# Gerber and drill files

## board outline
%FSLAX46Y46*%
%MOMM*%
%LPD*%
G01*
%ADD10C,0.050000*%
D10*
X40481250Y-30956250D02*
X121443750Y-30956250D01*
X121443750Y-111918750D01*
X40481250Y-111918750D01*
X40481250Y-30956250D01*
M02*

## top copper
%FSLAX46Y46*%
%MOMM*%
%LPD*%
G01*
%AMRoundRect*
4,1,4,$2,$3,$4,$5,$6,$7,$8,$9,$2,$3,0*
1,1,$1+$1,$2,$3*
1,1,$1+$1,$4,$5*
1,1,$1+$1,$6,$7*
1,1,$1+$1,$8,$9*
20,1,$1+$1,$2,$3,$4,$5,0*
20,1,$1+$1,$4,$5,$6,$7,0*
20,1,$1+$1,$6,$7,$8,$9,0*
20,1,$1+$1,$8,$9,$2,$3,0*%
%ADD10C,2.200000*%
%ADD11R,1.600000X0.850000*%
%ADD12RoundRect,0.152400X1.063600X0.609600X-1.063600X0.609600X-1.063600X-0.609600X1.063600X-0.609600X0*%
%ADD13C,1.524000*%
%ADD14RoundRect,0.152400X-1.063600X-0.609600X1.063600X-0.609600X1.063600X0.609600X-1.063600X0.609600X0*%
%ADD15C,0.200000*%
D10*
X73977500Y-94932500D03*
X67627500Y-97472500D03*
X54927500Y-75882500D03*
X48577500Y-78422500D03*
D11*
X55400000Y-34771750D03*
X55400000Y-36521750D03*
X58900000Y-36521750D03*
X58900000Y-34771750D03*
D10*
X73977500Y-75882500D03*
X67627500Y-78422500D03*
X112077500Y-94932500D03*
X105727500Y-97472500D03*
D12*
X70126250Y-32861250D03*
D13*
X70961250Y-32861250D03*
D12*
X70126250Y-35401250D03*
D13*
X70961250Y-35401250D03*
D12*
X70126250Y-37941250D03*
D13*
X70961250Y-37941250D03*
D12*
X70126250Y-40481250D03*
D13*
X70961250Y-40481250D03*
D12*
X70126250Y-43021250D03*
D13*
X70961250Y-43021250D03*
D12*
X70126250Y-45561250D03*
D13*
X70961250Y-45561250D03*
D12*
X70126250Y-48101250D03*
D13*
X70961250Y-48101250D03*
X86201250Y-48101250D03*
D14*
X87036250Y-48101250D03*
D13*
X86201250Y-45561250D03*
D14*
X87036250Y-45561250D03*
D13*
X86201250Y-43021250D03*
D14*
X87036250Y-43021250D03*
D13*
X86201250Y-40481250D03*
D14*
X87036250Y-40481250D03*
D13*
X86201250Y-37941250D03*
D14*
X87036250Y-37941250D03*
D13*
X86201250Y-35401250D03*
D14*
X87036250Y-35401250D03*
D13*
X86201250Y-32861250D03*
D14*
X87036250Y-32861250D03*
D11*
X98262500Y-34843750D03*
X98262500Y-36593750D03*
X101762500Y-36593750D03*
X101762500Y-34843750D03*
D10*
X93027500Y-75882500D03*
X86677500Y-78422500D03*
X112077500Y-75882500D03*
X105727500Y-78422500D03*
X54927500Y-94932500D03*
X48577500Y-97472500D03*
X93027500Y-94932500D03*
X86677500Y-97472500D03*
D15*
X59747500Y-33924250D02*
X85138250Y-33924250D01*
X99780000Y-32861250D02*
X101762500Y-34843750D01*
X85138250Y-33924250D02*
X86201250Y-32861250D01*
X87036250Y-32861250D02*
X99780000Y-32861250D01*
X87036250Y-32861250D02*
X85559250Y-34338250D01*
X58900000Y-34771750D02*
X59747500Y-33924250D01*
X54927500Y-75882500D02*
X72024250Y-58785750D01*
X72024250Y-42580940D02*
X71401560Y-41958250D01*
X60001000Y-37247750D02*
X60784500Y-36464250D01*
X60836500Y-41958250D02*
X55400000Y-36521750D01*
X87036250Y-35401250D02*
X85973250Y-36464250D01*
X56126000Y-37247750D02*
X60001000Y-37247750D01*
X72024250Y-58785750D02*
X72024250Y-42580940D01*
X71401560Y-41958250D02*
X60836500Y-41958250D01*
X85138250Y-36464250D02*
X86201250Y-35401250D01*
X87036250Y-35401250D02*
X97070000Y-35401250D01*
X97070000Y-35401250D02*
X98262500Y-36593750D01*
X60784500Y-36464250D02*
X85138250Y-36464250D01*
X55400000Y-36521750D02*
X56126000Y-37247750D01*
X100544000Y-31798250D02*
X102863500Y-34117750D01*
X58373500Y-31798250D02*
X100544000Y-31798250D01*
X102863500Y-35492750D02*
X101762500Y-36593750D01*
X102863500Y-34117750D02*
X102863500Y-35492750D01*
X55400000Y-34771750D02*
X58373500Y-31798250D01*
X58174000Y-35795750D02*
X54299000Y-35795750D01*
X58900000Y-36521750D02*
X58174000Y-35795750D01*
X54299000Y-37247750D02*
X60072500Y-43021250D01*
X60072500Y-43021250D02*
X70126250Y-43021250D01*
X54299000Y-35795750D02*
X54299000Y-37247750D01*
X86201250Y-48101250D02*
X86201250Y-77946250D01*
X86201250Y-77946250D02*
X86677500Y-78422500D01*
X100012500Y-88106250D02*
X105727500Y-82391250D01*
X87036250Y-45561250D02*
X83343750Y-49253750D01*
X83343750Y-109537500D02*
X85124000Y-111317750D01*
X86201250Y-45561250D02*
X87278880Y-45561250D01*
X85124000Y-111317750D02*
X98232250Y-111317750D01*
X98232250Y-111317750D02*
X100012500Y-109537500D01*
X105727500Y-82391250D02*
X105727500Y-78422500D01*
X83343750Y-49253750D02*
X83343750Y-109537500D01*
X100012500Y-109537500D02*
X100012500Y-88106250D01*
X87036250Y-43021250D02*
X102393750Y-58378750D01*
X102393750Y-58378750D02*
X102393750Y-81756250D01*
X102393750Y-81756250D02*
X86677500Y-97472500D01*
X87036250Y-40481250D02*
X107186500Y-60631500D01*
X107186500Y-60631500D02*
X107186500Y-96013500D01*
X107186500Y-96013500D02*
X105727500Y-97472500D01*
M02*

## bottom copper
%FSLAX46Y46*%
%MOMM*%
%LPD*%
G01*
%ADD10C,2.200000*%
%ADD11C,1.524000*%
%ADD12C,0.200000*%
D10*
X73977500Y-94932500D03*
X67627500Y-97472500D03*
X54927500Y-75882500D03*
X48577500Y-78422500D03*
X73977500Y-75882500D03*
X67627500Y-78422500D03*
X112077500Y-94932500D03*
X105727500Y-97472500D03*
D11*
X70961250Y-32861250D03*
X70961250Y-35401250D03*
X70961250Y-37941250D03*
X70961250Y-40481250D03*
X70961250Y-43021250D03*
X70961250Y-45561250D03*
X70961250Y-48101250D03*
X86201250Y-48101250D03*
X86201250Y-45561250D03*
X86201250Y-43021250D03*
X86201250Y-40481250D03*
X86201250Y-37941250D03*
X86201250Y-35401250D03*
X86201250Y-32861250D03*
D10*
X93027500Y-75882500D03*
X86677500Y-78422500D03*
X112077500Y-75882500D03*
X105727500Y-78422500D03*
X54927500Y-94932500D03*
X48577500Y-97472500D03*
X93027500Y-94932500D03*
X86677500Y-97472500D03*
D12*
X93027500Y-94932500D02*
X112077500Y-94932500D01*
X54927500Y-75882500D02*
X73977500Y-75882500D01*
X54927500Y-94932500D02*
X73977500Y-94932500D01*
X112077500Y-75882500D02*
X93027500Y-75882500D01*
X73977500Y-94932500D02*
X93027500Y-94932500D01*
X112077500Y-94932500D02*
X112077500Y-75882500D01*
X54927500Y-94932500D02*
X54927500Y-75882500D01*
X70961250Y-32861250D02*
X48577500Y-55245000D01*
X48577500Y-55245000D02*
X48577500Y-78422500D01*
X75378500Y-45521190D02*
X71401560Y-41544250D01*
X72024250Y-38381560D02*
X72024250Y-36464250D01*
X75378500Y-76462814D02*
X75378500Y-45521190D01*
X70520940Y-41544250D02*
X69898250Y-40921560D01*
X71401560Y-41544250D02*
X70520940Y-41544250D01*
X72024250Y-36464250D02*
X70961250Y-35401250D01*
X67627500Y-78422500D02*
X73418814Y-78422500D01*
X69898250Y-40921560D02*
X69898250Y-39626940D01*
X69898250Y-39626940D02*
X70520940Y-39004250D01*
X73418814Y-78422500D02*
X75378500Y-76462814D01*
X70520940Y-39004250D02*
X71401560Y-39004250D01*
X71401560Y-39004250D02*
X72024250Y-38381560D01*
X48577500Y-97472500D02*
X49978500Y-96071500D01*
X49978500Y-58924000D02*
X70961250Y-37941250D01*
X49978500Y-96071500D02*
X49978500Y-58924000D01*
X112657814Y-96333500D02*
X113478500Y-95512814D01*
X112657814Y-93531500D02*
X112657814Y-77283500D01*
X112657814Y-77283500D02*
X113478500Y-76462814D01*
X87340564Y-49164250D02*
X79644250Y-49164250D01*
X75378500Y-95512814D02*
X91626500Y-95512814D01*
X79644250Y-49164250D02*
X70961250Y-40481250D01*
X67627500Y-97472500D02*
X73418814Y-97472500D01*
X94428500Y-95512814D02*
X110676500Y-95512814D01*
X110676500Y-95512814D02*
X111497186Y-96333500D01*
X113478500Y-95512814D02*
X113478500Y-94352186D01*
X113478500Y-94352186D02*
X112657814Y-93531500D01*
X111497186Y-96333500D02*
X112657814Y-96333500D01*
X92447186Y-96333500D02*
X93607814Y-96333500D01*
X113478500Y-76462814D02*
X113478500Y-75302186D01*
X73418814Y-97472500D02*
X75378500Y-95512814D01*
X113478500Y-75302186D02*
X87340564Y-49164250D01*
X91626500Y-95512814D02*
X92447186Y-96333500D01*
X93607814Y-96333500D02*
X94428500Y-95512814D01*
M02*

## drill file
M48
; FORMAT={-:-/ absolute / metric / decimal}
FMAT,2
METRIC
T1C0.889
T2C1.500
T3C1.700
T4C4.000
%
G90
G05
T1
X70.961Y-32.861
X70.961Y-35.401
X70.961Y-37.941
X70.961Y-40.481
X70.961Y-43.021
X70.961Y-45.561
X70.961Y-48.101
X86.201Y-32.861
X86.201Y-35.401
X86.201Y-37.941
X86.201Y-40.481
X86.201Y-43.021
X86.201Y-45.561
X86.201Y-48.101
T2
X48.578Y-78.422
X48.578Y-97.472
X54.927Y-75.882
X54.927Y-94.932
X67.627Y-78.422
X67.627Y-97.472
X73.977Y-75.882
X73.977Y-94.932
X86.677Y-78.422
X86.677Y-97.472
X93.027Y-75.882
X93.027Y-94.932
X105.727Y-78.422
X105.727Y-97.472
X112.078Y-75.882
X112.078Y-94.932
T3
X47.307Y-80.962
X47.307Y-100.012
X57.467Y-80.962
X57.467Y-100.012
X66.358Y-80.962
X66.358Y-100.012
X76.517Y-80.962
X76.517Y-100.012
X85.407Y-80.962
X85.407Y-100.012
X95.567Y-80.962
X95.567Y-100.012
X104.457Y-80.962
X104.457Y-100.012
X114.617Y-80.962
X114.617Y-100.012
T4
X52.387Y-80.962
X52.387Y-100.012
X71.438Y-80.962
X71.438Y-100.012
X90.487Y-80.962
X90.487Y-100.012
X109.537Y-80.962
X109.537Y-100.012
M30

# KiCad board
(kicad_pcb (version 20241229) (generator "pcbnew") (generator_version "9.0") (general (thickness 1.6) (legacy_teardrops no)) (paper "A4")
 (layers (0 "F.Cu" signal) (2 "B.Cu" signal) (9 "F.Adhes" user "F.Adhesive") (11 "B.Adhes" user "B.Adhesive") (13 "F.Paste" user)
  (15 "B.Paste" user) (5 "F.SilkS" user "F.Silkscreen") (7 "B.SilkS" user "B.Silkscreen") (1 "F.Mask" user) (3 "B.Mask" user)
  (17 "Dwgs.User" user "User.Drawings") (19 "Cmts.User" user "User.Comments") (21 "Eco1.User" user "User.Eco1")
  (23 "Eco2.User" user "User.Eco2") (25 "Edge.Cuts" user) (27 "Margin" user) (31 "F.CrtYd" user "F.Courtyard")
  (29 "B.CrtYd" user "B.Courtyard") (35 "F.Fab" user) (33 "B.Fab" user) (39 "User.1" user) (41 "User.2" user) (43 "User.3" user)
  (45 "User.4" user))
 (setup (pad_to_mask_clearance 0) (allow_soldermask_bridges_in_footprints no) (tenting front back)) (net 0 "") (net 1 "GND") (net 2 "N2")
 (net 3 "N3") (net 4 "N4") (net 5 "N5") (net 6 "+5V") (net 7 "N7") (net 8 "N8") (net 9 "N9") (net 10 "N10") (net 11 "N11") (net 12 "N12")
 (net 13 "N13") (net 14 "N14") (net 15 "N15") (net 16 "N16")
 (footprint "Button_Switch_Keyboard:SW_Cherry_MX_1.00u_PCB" (layer "F.Cu") (at 73.9775 94.9325)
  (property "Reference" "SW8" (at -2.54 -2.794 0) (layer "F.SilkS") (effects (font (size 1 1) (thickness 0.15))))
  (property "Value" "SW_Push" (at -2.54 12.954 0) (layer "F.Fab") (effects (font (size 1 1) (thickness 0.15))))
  (pad "" np_thru_hole circle (at -7.62 5.08) (size 1.7 1.7) (drill 1.7) (layers "*.Cu" "*.Mask"))
  (pad "" np_thru_hole circle (at -2.54 5.08) (size 4 4) (drill 4) (layers "*.Cu" "*.Mask"))
  (pad "" np_thru_hole circle (at 2.54 5.08) (size 1.7 1.7) (drill 1.7) (layers "*.Cu" "*.Mask"))
  (pad "1" thru_hole circle (at 0 0) (size 2.2 2.2) (drill 1.5) (layers "*.Cu" "*.Mask") (remove_unused_layers no) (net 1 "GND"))
  (pad "2" thru_hole circle (at -6.35 2.54) (size 2.2 2.2) (drill 1.5) (layers "*.Cu" "*.Mask") (remove_unused_layers no) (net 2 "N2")))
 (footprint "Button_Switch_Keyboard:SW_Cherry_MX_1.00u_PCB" (layer "F.Cu") (at 54.9275 75.8825)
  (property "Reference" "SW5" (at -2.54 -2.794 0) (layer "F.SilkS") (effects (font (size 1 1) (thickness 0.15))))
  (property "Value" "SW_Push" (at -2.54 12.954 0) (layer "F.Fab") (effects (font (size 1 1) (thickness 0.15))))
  (pad "" np_thru_hole circle (at -7.62 5.08) (size 1.7 1.7) (drill 1.7) (layers "*.Cu" "*.Mask"))
  (pad "" np_thru_hole circle (at -2.54 5.08) (size 4 4) (drill 4) (layers "*.Cu" "*.Mask"))
  (pad "" np_thru_hole circle (at 2.54 5.08) (size 1.7 1.7) (drill 1.7) (layers "*.Cu" "*.Mask"))
  (pad "1" thru_hole circle (at 0 0) (size 2.2 2.2) (drill 1.5) (layers "*.Cu" "*.Mask") (remove_unused_layers no) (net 1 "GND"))
  (pad "2" thru_hole circle (at -6.35 2.54) (size 2.2 2.2) (drill 1.5) (layers "*.Cu" "*.Mask") (remove_unused_layers no) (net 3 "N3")))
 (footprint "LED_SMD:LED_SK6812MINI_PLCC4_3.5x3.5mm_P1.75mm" (layer "F.Cu") (at 57.15 35.64675)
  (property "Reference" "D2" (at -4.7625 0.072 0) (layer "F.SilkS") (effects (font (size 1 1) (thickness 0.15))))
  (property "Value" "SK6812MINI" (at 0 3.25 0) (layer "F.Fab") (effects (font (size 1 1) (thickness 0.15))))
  (pad "1" smd rect (at -1.75 -0.875) (size 1.6 0.85) (layers "F.Cu" "F.Mask" "F.Paste") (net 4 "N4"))
  (pad "2" smd rect (at -1.75 0.875) (size 1.6 0.85) (layers "F.Cu" "F.Mask" "F.Paste") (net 1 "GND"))
  (pad "3" smd rect (at 1.75 0.875) (size 1.6 0.85) (layers "F.Cu" "F.Mask" "F.Paste") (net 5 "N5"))
  (pad "4" smd rect (at 1.75 -0.875) (size 1.6 0.85) (layers "F.Cu" "F.Mask" "F.Paste") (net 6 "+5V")))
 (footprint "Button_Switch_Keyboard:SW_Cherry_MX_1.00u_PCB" (layer "F.Cu") (at 73.9775 75.8825)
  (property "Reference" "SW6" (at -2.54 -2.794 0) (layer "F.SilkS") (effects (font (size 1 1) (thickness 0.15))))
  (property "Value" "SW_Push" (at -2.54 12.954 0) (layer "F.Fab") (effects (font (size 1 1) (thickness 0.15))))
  (pad "" np_thru_hole circle (at -7.62 5.08) (size 1.7 1.7) (drill 1.7) (layers "*.Cu" "*.Mask"))
  (pad "" np_thru_hole circle (at -2.54 5.08) (size 4 4) (drill 4) (layers "*.Cu" "*.Mask"))
  (pad "" np_thru_hole circle (at 2.54 5.08) (size 1.7 1.7) (drill 1.7) (layers "*.Cu" "*.Mask"))
  (pad "1" thru_hole circle (at 0 0) (size 2.2 2.2) (drill 1.5) (layers "*.Cu" "*.Mask") (remove_unused_layers no) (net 1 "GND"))
  (pad "2" thru_hole circle (at -6.35 2.54) (size 2.2 2.2) (drill 1.5) (layers "*.Cu" "*.Mask") (remove_unused_layers no) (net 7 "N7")))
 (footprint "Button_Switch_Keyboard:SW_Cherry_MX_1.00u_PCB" (layer "F.Cu") (at 112.0775 94.9325)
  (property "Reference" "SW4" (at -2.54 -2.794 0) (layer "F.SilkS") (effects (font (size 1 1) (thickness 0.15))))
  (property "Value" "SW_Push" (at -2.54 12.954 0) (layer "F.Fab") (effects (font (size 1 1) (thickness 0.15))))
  (pad "" np_thru_hole circle (at -7.62 5.08) (size 1.7 1.7) (drill 1.7) (layers "*.Cu" "*.Mask"))
  (pad "" np_thru_hole circle (at -2.54 5.08) (size 4 4) (drill 4) (layers "*.Cu" "*.Mask"))
  (pad "" np_thru_hole circle (at 2.54 5.08) (size 1.7 1.7) (drill 1.7) (layers "*.Cu" "*.Mask"))
  (pad "1" thru_hole circle (at 0 0) (size 2.2 2.2) (drill 1.5) (layers "*.Cu" "*.Mask") (remove_unused_layers no) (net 1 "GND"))
  (pad "2" thru_hole circle (at -6.35 2.54) (size 2.2 2.2) (drill 1.5) (layers "*.Cu" "*.Mask") (remove_unused_layers no) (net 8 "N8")))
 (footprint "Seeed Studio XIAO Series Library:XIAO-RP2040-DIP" (layer "F.Cu") (at 78.58125 40.48125)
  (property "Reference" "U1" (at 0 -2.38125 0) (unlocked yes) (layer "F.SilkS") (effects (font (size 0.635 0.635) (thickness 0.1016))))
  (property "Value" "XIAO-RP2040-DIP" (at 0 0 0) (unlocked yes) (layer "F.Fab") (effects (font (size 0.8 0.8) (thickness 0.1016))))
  (pad "1" smd roundrect (at -8.455 -7.62 180) (size 2.432 1.524) (layers "F.Cu" "F.Mask") (roundrect_rratio 0.1) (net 3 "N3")
   (thermal_bridge_angle 45))
  (pad "1" thru_hole circle (at -7.62 -7.62 180) (size 1.524 1.524) (drill 0.889) (layers "*.Cu" "*.Mask") (remove_unused_layers no)
   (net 3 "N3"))
  (pad "2" smd roundrect (at -8.455 -5.08 180) (size 2.432 1.524) (layers "F.Cu" "F.Mask") (roundrect_rratio 0.1) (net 7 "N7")
   (thermal_bridge_angle 45))
  (pad "2" thru_hole circle (at -7.62 -5.08 180) (size 1.524 1.524) (drill 0.889) (layers "*.Cu" "*.Mask") (remove_unused_layers no)
   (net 7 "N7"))
  (pad "3" smd roundrect (at -8.455 -2.54 180) (size 2.432 1.524) (layers "F.Cu" "F.Mask") (roundrect_rratio 0.1) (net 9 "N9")
   (thermal_bridge_angle 45))
  (pad "3" thru_hole circle (at -7.62 -2.54 180) (size 1.524 1.524) (drill 0.889) (layers "*.Cu" "*.Mask") (remove_unused_layers no)
   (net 9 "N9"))
  (pad "4" smd roundrect (at -8.455 0 180) (size 2.432 1.524) (layers "F.Cu" "F.Mask") (roundrect_rratio 0.1) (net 2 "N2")
   (thermal_bridge_angle 45))
  (pad "4" thru_hole circle (at -7.62 0 180) (size 1.524 1.524) (drill 0.889) (layers "*.Cu" "*.Mask") (remove_unused_layers no)
   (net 2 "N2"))
  (pad "5" smd roundrect (at -8.455 2.54 180) (size 2.432 1.524) (layers "F.Cu" "F.Mask") (roundrect_rratio 0.1) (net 5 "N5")
   (thermal_bridge_angle 45))
  (pad "5" thru_hole circle (at -7.62 2.54 180) (size 1.524 1.524) (drill 0.889) (layers "*.Cu" "*.Mask") (remove_unused_layers no)
   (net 5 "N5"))
  (pad "6" smd roundrect (at -8.455 5.08 180) (size 2.432 1.524) (layers "F.Cu" "F.Mask") (roundrect_rratio 0.1) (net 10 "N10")
   (thermal_bridge_angle 45))
  (pad "6" thru_hole circle (at -7.62 5.08 180) (size 1.524 1.524) (drill 0.889) (layers "*.Cu" "*.Mask") (remove_unused_layers no)
   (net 10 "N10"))
  (pad "7" smd roundrect (at -8.455 7.62 180) (size 2.432 1.524) (layers "F.Cu" "F.Mask") (roundrect_rratio 0.1) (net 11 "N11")
   (thermal_bridge_angle 45))
  (pad "7" thru_hole circle (at -7.62 7.62 180) (size 1.524 1.524) (drill 0.889) (layers "*.Cu" "*.Mask") (remove_unused_layers no)
   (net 11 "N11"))
  (pad "8" thru_hole circle (at 7.62 7.62) (size 1.524 1.524) (drill 0.889) (layers "*.Cu" "*.Mask") (remove_unused_layers no)
   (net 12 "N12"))
  (pad "8" smd roundrect (at 8.455 7.62) (size 2.432 1.524) (layers "F.Cu" "F.Mask") (roundrect_rratio 0.1) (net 12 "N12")
   (thermal_bridge_angle 45))
  (pad "9" thru_hole circle (at 7.62 5.08) (size 1.524 1.524) (drill 0.889) (layers "*.Cu" "*.Mask") (remove_unused_layers no)
   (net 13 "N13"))
  (pad "9" smd roundrect (at 8.455 5.08) (size 2.432 1.524) (layers "F.Cu" "F.Mask") (roundrect_rratio 0.1) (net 13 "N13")
   (thermal_bridge_angle 45))
  (pad "10" thru_hole circle (at 7.62 2.54) (size 1.524 1.524) (drill 0.889) (layers "*.Cu" "*.Mask") (remove_unused_layers no)
   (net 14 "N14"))
  (pad "10" smd roundrect (at 8.455 2.54) (size 2.432 1.524) (layers "F.Cu" "F.Mask") (roundrect_rratio 0.1) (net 14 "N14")
   (thermal_bridge_angle 45))
  (pad "11" thru_hole circle (at 7.62 0) (size 1.524 1.524) (drill 0.889) (layers "*.Cu" "*.Mask") (remove_unused_layers no) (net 8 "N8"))
  (pad "11" smd roundrect (at 8.455 0) (size 2.432 1.524) (layers "F.Cu" "F.Mask") (roundrect_rratio 0.1) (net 8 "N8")
   (thermal_bridge_angle 45))
  (pad "12" thru_hole circle (at 7.62 -2.54) (size 1.524 1.524) (drill 0.889) (layers "*.Cu" "*.Mask") (remove_unused_layers no)
   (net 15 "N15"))
  (pad "12" smd roundrect (at 8.455 -2.54) (size 2.432 1.524) (layers "F.Cu" "F.Mask") (roundrect_rratio 0.1) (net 15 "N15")
   (thermal_bridge_angle 45))
  (pad "13" thru_hole circle (at 7.62 -5.08) (size 1.524 1.524) (drill 0.889) (layers "*.Cu" "*.Mask") (remove_unused_layers no)
   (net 1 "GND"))
  (pad "13" smd roundrect (at 8.455 -5.08) (size 2.432 1.524) (layers "F.Cu" "F.Mask") (roundrect_rratio 0.1) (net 1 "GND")
   (thermal_bridge_angle 45))
  (pad "14" thru_hole circle (at 7.62 -7.62) (size 1.524 1.524) (drill 0.889) (layers "*.Cu" "*.Mask") (remove_unused_layers no)
   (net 6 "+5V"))
  (pad "14" smd roundrect (at 8.455 -7.62) (size 2.432 1.524) (layers "F.Cu" "F.Mask") (roundrect_rratio 0.1) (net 6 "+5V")
   (thermal_bridge_angle 45)))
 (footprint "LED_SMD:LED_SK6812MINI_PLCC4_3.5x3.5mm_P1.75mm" (layer "F.Cu") (at 100.0125 35.71875)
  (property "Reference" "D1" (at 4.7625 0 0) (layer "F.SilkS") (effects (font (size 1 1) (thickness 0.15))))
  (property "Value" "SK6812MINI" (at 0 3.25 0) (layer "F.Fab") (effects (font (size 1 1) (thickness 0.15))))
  (pad "1" smd rect (at -1.75 -0.875) (size 1.6 0.85) (layers "F.Cu" "F.Mask" "F.Paste") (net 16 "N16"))
  (pad "2" smd rect (at -1.75 0.875) (size 1.6 0.85) (layers "F.Cu" "F.Mask" "F.Paste") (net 1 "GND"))
  (pad "3" smd rect (at 1.75 0.875) (size 1.6 0.85) (layers "F.Cu" "F.Mask" "F.Paste") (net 4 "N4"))
  (pad "4" smd rect (at 1.75 -0.875) (size 1.6 0.85) (layers "F.Cu" "F.Mask" "F.Paste") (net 6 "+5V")))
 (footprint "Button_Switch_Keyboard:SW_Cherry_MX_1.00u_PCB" (layer "F.Cu") (at 93.0275 75.8825)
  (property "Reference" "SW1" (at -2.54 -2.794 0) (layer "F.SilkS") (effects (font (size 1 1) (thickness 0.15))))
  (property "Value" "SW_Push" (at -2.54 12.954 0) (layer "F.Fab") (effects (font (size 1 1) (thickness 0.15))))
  (pad "" np_thru_hole circle (at -7.62 5.08) (size 1.7 1.7) (drill 1.7) (layers "*.Cu" "*.Mask"))
  (pad "" np_thru_hole circle (at -2.54 5.08) (size 4 4) (drill 4) (layers "*.Cu" "*.Mask"))
  (pad "" np_thru_hole circle (at 2.54 5.08) (size 1.7 1.7) (drill 1.7) (layers "*.Cu" "*.Mask"))
  (pad "1" thru_hole circle (at 0 0) (size 2.2 2.2) (drill 1.5) (layers "*.Cu" "*.Mask") (remove_unused_layers no) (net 1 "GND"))
  (pad "2" thru_hole circle (at -6.35 2.54) (size 2.2 2.2) (drill 1.5) (layers "*.Cu" "*.Mask") (remove_unused_layers no) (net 12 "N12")))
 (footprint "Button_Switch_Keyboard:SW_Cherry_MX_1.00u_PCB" (layer "F.Cu") (at 112.0775 75.8825)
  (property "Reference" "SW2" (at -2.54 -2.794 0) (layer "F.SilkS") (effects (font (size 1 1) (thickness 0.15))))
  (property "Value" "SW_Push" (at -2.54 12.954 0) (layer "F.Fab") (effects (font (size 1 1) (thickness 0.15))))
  (pad "" np_thru_hole circle (at -7.62 5.08) (size 1.7 1.7) (drill 1.7) (layers "*.Cu" "*.Mask"))
  (pad "" np_thru_hole circle (at -2.54 5.08) (size 4 4) (drill 4) (layers "*.Cu" "*.Mask"))
  (pad "" np_thru_hole circle (at 2.54 5.08) (size 1.7 1.7) (drill 1.7) (layers "*.Cu" "*.Mask"))
  (pad "1" thru_hole circle (at 0 0) (size 2.2 2.2) (drill 1.5) (layers "*.Cu" "*.Mask") (remove_unused_layers no) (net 1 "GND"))
  (pad "2" thru_hole circle (at -6.35 2.54) (size 2.2 2.2) (drill 1.5) (layers "*.Cu" "*.Mask") (remove_unused_layers no) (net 13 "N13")))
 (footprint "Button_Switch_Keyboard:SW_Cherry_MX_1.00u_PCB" (layer "F.Cu") (at 54.9275 94.9325)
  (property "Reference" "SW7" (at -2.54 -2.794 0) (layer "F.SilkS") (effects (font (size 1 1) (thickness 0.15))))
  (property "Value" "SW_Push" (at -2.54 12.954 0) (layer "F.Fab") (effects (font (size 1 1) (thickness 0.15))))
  (pad "" np_thru_hole circle (at -7.62 5.08) (size 1.7 1.7) (drill 1.7) (layers "*.Cu" "*.Mask"))
  (pad "" np_thru_hole circle (at -2.54 5.08) (size 4 4) (drill 4) (layers "*.Cu" "*.Mask"))
  (pad "" np_thru_hole circle (at 2.54 5.08) (size 1.7 1.7) (drill 1.7) (layers "*.Cu" "*.Mask"))
  (pad "1" thru_hole circle (at 0 0) (size 2.2 2.2) (drill 1.5) (layers "*.Cu" "*.Mask") (remove_unused_layers no) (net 1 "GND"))
  (pad "2" thru_hole circle (at -6.35 2.54) (size 2.2 2.2) (drill 1.5) (layers "*.Cu" "*.Mask") (remove_unused_layers no) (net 9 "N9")))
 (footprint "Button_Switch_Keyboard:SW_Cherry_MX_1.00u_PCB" (layer "F.Cu") (at 93.0275 94.9325)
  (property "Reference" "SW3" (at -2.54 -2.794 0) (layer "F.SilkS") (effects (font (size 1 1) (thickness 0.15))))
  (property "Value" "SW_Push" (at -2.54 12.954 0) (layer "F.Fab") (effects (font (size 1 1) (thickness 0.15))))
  (pad "" np_thru_hole circle (at -7.62 5.08) (size 1.7 1.7) (drill 1.7) (layers "*.Cu" "*.Mask"))
  (pad "" np_thru_hole circle (at -2.54 5.08) (size 4 4) (drill 4) (layers "*.Cu" "*.Mask"))
  (pad "" np_thru_hole circle (at 2.54 5.08) (size 1.7 1.7) (drill 1.7) (layers "*.Cu" "*.Mask"))
  (pad "1" thru_hole circle (at 0 0) (size 2.2 2.2) (drill 1.5) (layers "*.Cu" "*.Mask") (remove_unused_layers no) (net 1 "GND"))
  (pad "2" thru_hole circle (at -6.35 2.54) (size 2.2 2.2) (drill 1.5) (layers "*.Cu" "*.Mask") (remove_unused_layers no) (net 14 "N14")))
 (gr_rect (start 40.48125 30.95625) (end 121.44375 111.91875) (stroke (width 0.05) (type default)) (fill no) (layer "Edge.Cuts"))
 (segment (start 59.7475 33.92425) (end 85.13825 33.92425) (width 0.2) (layer "F.Cu") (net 6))
 (segment (start 99.78 32.86125) (end 101.7625 34.84375) (width 0.2) (layer "F.Cu") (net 6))
 (segment (start 85.13825 33.92425) (end 86.20125 32.86125) (width 0.2) (layer "F.Cu") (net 6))
 (segment (start 87.03625 32.86125) (end 99.78 32.86125) (width 0.2) (layer "F.Cu") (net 6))
 (segment (start 87.03625 32.86125) (end 85.55925 34.33825) (width 0.2) (layer "F.Cu") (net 6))
 (segment (start 58.9 34.77175) (end 59.7475 33.92425) (width 0.2) (layer "F.Cu") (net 6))
 (segment (start 54.9275 75.8825) (end 72.02425 58.78575) (width 0.2) (layer "F.Cu") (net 1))
 (segment (start 72.02425 42.58094) (end 71.40156 41.95825) (width 0.2) (layer "F.Cu") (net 1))
 (segment (start 60.001 37.24775) (end 60.7845 36.46425) (width 0.2) (layer "F.Cu") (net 1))
 (segment (start 60.8365 41.95825) (end 55.4 36.52175) (width 0.2) (layer "F.Cu") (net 1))
 (segment (start 87.03625 35.40125) (end 85.97325 36.46425) (width 0.2) (layer "F.Cu") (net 1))
 (segment (start 56.126 37.24775) (end 60.001 37.24775) (width 0.2) (layer "F.Cu") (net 1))
 (segment (start 72.02425 58.78575) (end 72.02425 42.58094) (width 0.2) (layer "F.Cu") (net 1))
 (segment (start 71.40156 41.95825) (end 60.8365 41.95825) (width 0.2) (layer "F.Cu") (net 1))
 (segment (start 85.13825 36.46425) (end 86.20125 35.40125) (width 0.2) (layer "F.Cu") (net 1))
 (segment (start 87.03625 35.40125) (end 97.07 35.40125) (width 0.2) (layer "F.Cu") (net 1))
 (segment (start 97.07 35.40125) (end 98.2625 36.59375) (width 0.2) (layer "F.Cu") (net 1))
 (segment (start 60.7845 36.46425) (end 85.13825 36.46425) (width 0.2) (layer "F.Cu") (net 1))
 (segment (start 55.4 36.52175) (end 56.126 37.24775) (width 0.2) (layer "F.Cu") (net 1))
 (segment (start 93.0275 94.9325) (end 112.0775 94.9325) (width 0.2) (layer "B.Cu") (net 1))
 (segment (start 54.9275 75.8825) (end 73.9775 75.8825) (width 0.2) (layer "B.Cu") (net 1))
 (segment (start 54.9275 94.9325) (end 73.9775 94.9325) (width 0.2) (layer "B.Cu") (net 1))
 (segment (start 112.0775 75.8825) (end 93.0275 75.8825) (width 0.2) (layer "B.Cu") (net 1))
 (segment (start 73.9775 94.9325) (end 93.0275 94.9325) (width 0.2) (layer "B.Cu") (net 1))
 (segment (start 112.0775 94.9325) (end 112.0775 75.8825) (width 0.2) (layer "B.Cu") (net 1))
 (segment (start 54.9275 94.9325) (end 54.9275 75.8825) (width 0.2) (layer "B.Cu") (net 1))
 (segment (start 100.544 31.79825) (end 102.8635 34.11775) (width 0.2) (layer "F.Cu") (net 4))
 (segment (start 58.3735 31.79825) (end 100.544 31.79825) (width 0.2) (layer "F.Cu") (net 4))
 (segment (start 102.8635 35.49275) (end 101.7625 36.59375) (width 0.2) (layer "F.Cu") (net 4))
 (segment (start 102.8635 34.11775) (end 102.8635 35.49275) (width 0.2) (layer "F.Cu") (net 4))
 (segment (start 55.4 34.77175) (end 58.3735 31.79825) (width 0.2) (layer "F.Cu") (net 4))
 (segment (start 58.174 35.79575) (end 54.299 35.79575) (width 0.2) (layer "F.Cu") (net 5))
 (segment (start 58.9 36.52175) (end 58.174 35.79575) (width 0.2) (layer "F.Cu") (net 5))
 (segment (start 54.299 37.24775) (end 60.0725 43.02125) (width 0.2) (layer "F.Cu") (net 5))
 (segment (start 60.0725 43.02125) (end 70.12625 43.02125) (width 0.2) (layer "F.Cu") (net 5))
 (segment (start 54.299 35.79575) (end 54.299 37.24775) (width 0.2) (layer "F.Cu") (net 5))
 (segment (start 86.20125 48.10125) (end 86.20125 77.94625) (width 0.2) (layer "F.Cu") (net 12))
 (segment (start 86.20125 77.94625) (end 86.6775 78.4225) (width 0.2) (layer "F.Cu") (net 12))
 (segment (start 100.0125 88.10625) (end 105.7275 82.39125) (width 0.2) (layer "F.Cu") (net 13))
 (segment (start 87.03625 45.56125) (end 83.34375 49.25375) (width 0.2) (layer "F.Cu") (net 13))
 (segment (start 83.34375 109.5375) (end 85.124 111.31775) (width 0.2) (layer "F.Cu") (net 13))
 (segment (start 86.20125 45.56125) (end 87.27888 45.56125) (width 0.2) (layer "F.Cu") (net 13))
 (segment (start 85.124 111.31775) (end 98.23225 111.31775) (width 0.2) (layer "F.Cu") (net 13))
 (segment (start 98.23225 111.31775) (end 100.0125 109.5375) (width 0.2) (layer "F.Cu") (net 13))
 (segment (start 105.7275 82.39125) (end 105.7275 78.4225) (width 0.2) (layer "F.Cu") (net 13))
 (segment (start 83.34375 49.25375) (end 83.34375 109.5375) (width 0.2) (layer "F.Cu") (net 13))
 (segment (start 100.0125 109.5375) (end 100.0125 88.10625) (width 0.2) (layer "F.Cu") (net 13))
 (segment (start 87.03625 43.02125) (end 102.39375 58.37875) (width 0.2) (layer "F.Cu") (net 14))
 (segment (start 102.39375 58.37875) (end 102.39375 81.75625) (width 0.2) (layer "F.Cu") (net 14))
 (segment (start 102.39375 81.75625) (end 86.6775 97.4725) (width 0.2) (layer "F.Cu") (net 14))
 (segment (start 87.03625 40.48125) (end 107.1865 60.6315) (width 0.2) (layer "F.Cu") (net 8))
 (segment (start 107.1865 60.6315) (end 107.1865 96.0135) (width 0.2) (layer "F.Cu") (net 8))
 (segment (start 107.1865 96.0135) (end 105.7275 97.4725) (width 0.2) (layer "F.Cu") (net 8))
 (segment (start 70.96125 32.86125) (end 48.5775 55.245) (width 0.2) (layer "B.Cu") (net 3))
 (segment (start 48.5775 55.245) (end 48.5775 78.4225) (width 0.2) (layer "B.Cu") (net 3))
 (segment (start 75.3785 45.52119) (end 71.40156 41.54425) (width 0.2) (layer "B.Cu") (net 7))
 (segment (start 72.02425 38.38156) (end 72.02425 36.46425) (width 0.2) (layer "B.Cu") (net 7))
 (segment (start 75.3785 76.462814) (end 75.3785 45.52119) (width 0.2) (layer "B.Cu") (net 7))
 (segment (start 70.52094 41.54425) (end 69.89825 40.92156) (width 0.2) (layer "B.Cu") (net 7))
 (segment (start 71.40156 41.54425) (end 70.52094 41.54425) (width 0.2) (layer "B.Cu") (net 7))
 (segment (start 72.02425 36.46425) (end 70.96125 35.40125) (width 0.2) (layer "B.Cu") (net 7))
 (segment (start 67.6275 78.4225) (end 73.418814 78.4225) (width 0.2) (layer "B.Cu") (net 7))
 (segment (start 69.89825 40.92156) (end 69.89825 39.62694) (width 0.2) (layer "B.Cu") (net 7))
 (segment (start 69.89825 39.62694) (end 70.52094 39.00425) (width 0.2) (layer "B.Cu") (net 7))
 (segment (start 73.418814 78.4225) (end 75.3785 76.462814) (width 0.2) (layer "B.Cu") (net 7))
 (segment (start 70.52094 39.00425) (end 71.40156 39.00425) (width 0.2) (layer "B.Cu") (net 7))
 (segment (start 71.40156 39.00425) (end 72.02425 38.38156) (width 0.2) (layer "B.Cu") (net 7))
 (segment (start 48.5775 97.4725) (end 49.9785 96.0715) (width 0.2) (layer "B.Cu") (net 9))
 (segment (start 49.9785 58.924) (end 70.96125 37.94125) (width 0.2) (layer "B.Cu") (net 9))
 (segment (start 49.9785 96.0715) (end 49.9785 58.924) (width 0.2) (layer "B.Cu") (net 9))
 (segment (start 112.657814 96.3335) (end 113.4785 95.512814) (width 0.2) (layer "B.Cu") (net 2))
 (segment (start 112.657814 93.5315) (end 112.657814 77.2835) (width 0.2) (layer "B.Cu") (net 2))
 (segment (start 112.657814 77.2835) (end 113.4785 76.462814) (width 0.2) (layer "B.Cu") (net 2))
 (segment (start 87.340564 49.16425) (end 79.64425 49.16425) (width 0.2) (layer "B.Cu") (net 2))
 (segment (start 75.3785 95.512814) (end 91.6265 95.512814) (width 0.2) (layer "B.Cu") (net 2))
 (segment (start 79.64425 49.16425) (end 70.96125 40.48125) (width 0.2) (layer "B.Cu") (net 2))
 (segment (start 67.6275 97.4725) (end 73.418814 97.4725) (width 0.2) (layer "B.Cu") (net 2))
 (segment (start 94.4285 95.512814) (end 110.6765 95.512814) (width 0.2) (layer "B.Cu") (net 2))
 (segment (start 110.6765 95.512814) (end 111.497186 96.3335) (width 0.2) (layer "B.Cu") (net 2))
 (segment (start 113.4785 95.512814) (end 113.4785 94.352186) (width 0.2) (layer "B.Cu") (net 2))
 (segment (start 113.4785 94.352186) (end 112.657814 93.5315) (width 0.2) (layer "B.Cu") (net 2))
 (segment (start 111.497186 96.3335) (end 112.657814 96.3335) (width 0.2) (layer "B.Cu") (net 2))
 (segment (start 92.447186 96.3335) (end 93.607814 96.3335) (width 0.2) (layer "B.Cu") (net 2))
 (segment (start 113.4785 76.462814) (end 113.4785 75.302186) (width 0.2) (layer "B.Cu") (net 2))
 (segment (start 73.418814 97.4725) (end 75.3785 95.512814) (width 0.2) (layer "B.Cu") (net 2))
 (segment (start 113.4785 75.302186) (end 87.340564 49.16425) (width 0.2) (layer "B.Cu") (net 2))
 (segment (start 91.6265 95.512814) (end 92.447186 96.3335) (width 0.2) (layer "B.Cu") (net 2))
 (segment (start 93.607814 96.3335) (end 94.4285 95.512814) (width 0.2) (layer "B.Cu") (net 2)))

